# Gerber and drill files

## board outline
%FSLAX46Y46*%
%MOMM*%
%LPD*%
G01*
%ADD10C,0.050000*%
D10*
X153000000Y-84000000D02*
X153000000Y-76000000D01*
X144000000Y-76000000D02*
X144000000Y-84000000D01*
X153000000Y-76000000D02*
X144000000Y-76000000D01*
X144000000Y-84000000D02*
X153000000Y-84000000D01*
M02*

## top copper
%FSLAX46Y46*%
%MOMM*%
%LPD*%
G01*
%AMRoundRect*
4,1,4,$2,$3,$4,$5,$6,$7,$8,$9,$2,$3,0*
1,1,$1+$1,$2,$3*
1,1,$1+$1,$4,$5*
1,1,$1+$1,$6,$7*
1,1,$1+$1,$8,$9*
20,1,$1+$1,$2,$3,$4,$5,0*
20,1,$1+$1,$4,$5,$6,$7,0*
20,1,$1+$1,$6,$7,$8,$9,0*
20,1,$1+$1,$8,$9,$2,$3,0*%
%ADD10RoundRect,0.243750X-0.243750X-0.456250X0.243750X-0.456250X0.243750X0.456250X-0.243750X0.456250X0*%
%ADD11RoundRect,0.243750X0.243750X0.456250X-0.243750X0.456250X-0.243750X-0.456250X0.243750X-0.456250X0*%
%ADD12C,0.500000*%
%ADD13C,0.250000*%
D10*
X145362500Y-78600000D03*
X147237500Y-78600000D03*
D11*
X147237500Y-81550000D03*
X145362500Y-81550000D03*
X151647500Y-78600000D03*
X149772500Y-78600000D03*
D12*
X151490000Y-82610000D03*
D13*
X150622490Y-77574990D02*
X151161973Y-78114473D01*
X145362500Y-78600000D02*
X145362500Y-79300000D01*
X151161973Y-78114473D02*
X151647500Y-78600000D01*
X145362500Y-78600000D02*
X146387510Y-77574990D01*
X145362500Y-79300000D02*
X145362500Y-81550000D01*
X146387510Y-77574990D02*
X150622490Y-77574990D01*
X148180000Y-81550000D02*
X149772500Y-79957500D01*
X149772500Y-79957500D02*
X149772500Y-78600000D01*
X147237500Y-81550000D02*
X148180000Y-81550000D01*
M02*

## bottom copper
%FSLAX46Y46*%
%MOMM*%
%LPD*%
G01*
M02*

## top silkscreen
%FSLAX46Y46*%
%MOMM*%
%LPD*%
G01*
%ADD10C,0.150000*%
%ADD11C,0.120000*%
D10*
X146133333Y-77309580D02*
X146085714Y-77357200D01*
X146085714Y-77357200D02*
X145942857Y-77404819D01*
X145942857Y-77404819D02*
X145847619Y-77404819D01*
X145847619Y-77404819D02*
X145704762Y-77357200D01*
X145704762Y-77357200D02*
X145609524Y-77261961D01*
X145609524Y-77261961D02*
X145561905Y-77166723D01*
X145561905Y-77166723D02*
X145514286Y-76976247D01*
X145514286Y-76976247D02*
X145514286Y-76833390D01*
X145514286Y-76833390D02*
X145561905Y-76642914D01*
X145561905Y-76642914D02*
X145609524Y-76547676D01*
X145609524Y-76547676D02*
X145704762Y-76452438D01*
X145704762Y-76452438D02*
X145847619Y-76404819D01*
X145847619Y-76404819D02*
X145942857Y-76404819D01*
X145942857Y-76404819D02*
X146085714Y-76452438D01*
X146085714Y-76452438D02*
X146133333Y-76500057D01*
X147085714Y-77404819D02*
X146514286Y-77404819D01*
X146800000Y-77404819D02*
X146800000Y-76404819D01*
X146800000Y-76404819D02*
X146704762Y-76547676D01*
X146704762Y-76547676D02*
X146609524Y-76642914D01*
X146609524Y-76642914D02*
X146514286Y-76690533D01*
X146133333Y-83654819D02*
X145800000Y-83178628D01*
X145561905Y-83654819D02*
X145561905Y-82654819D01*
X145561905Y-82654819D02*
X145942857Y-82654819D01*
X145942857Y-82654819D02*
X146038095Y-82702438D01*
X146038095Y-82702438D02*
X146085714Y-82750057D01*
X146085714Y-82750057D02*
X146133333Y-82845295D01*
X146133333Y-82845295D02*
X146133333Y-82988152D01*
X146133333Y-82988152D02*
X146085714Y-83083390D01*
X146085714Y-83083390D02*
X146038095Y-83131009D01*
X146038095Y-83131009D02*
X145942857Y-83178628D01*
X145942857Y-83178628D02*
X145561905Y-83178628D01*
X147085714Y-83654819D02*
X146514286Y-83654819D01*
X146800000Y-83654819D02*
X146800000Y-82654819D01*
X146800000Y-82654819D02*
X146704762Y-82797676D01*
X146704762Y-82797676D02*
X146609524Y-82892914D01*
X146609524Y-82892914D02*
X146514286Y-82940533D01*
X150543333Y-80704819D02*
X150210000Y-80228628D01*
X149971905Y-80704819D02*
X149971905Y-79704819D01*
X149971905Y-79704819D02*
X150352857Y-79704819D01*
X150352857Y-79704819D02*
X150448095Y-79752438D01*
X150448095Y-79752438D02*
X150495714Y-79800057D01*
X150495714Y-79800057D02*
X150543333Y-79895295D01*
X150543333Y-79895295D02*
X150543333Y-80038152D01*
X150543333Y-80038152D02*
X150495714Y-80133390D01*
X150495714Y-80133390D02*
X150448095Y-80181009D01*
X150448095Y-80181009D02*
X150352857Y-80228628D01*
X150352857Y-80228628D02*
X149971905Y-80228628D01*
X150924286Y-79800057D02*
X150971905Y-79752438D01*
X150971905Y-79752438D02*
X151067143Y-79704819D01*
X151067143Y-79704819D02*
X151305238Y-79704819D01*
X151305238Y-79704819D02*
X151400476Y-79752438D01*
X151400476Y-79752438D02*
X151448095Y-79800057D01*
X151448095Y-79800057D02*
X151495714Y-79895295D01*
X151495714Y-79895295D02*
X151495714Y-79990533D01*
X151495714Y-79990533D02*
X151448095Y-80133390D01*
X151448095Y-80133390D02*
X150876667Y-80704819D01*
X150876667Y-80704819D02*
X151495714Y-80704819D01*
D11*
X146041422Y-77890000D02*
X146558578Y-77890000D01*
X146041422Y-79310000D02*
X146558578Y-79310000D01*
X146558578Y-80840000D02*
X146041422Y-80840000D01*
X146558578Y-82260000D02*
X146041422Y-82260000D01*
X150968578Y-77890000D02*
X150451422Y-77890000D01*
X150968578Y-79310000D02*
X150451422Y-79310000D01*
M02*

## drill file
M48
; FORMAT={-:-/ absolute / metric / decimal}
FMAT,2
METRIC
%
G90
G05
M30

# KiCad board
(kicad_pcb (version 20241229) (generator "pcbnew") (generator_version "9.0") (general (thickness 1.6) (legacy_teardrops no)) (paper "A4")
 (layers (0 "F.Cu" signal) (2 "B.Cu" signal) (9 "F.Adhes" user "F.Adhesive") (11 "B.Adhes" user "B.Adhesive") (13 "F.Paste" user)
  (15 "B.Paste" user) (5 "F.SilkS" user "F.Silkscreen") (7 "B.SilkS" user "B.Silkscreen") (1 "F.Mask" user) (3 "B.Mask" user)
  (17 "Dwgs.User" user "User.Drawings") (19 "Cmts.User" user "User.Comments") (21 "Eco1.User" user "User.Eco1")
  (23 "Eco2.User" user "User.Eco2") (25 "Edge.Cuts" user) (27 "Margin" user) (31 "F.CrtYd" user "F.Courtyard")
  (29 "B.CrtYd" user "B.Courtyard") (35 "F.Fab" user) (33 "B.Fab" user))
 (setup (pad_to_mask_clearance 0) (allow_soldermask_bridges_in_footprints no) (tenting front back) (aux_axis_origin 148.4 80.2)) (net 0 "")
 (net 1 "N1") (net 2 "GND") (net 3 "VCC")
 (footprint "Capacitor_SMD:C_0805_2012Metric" (layer "F.Cu") (at 146.3 78.6)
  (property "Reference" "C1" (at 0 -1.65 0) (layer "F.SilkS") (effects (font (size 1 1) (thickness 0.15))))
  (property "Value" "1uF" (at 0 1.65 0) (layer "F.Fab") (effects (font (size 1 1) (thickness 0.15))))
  (fp_line (start -0.258578 -0.71) (end 0.258578 -0.71) (stroke (width 0.12) (type solid)) (layer "F.SilkS"))
  (fp_line (start -0.258578 0.71) (end 0.258578 0.71) (stroke (width 0.12) (type solid)) (layer "F.SilkS"))
  (pad "1" smd roundrect (at -0.9375 0) (size 0.975 1.4) (layers "F.Cu" "F.Mask" "F.Paste") (roundrect_rratio 0.25) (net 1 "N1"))
  (pad "2" smd roundrect (at 0.9375 0) (size 0.975 1.4) (layers "F.Cu" "F.Mask" "F.Paste") (roundrect_rratio 0.25) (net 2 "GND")))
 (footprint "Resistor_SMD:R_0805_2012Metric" (layer "F.Cu") (at 146.3 81.55 180)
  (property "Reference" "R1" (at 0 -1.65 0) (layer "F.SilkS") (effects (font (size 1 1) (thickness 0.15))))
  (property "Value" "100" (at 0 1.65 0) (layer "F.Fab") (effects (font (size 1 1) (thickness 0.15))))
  (fp_line (start -0.258578 0.71) (end 0.258578 0.71) (stroke (width 0.12) (type solid)) (layer "F.SilkS"))
  (fp_line (start -0.258578 -0.71) (end 0.258578 -0.71) (stroke (width 0.12) (type solid)) (layer "F.SilkS"))
  (pad "1" smd roundrect (at -0.9375 0 180) (size 0.975 1.4) (layers "F.Cu" "F.Mask" "F.Paste") (roundrect_rratio 0.25) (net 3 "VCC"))
  (pad "2" smd roundrect (at 0.9375 0 180) (size 0.975 1.4) (layers "F.Cu" "F.Mask" "F.Paste") (roundrect_rratio 0.25) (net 1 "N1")))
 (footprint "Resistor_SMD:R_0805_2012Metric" (layer "F.Cu") (at 150.71 78.6 180)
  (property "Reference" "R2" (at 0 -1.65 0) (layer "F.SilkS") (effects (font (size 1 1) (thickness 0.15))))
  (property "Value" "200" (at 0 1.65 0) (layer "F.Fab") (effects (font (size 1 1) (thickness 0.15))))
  (fp_line (start -0.258578 0.71) (end 0.258578 0.71) (stroke (width 0.12) (type solid)) (layer "F.SilkS"))
  (fp_line (start -0.258578 -0.71) (end 0.258578 -0.71) (stroke (width 0.12) (type solid)) (layer "F.SilkS"))
  (pad "1" smd roundrect (at -0.9375 0 180) (size 0.975 1.4) (layers "F.Cu" "F.Mask" "F.Paste") (roundrect_rratio 0.25) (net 1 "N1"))
  (pad "2" smd roundrect (at 0.9375 0 180) (size 0.975 1.4) (layers "F.Cu" "F.Mask" "F.Paste") (roundrect_rratio 0.25) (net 3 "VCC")))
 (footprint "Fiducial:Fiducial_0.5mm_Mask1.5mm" (layer "F.Cu") (at 151.49 82.61)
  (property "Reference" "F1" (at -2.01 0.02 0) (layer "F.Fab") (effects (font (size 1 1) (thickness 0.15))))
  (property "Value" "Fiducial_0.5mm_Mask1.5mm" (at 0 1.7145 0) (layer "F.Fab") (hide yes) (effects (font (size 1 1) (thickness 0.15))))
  (pad "" smd circle (at 0 0) (size 0.5 0.5) (layers "F.Cu" "F.Mask") (solder_mask_margin 0.5) (clearance 0.5)))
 (gr_line (start 153 84) (end 153 76) (stroke (width 0.05) (type solid)) (layer "Edge.Cuts"))
 (gr_line (start 144 76) (end 144 84) (stroke (width 0.05) (type solid)) (layer "Edge.Cuts"))
 (gr_line (start 153 76) (end 144 76) (stroke (width 0.05) (type solid)) (layer "Edge.Cuts"))
 (gr_line (start 144 84) (end 153 84) (stroke (width 0.05) (type solid)) (layer "Edge.Cuts"))
 (segment (start 150.62249 77.57499) (end 151.161973 78.114473) (width 0.25) (layer "F.Cu") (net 1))
 (segment (start 145.3625 78.6) (end 145.3625 79.3) (width 0.25) (layer "F.Cu") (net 1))
 (segment (start 151.161973 78.114473) (end 151.6475 78.6) (width 0.25) (layer "F.Cu") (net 1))
 (segment (start 145.3625 78.6) (end 146.38751 77.57499) (width 0.25) (layer "F.Cu") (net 1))
 (segment (start 145.3625 79.3) (end 145.3625 81.55) (width 0.25) (layer "F.Cu") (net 1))
 (segment (start 146.38751 77.57499) (end 150.62249 77.57499) (width 0.25) (layer "F.Cu") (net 1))
 (segment (start 148.18 81.55) (end 149.7725 79.9575) (width 0.25) (layer "F.Cu") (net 3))
 (segment (start 149.7725 79.9575) (end 149.7725 78.6) (width 0.25) (layer "F.Cu") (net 3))
 (segment (start 147.2375 81.55) (end 148.18 81.55) (width 0.25) (layer "F.Cu") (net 3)))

